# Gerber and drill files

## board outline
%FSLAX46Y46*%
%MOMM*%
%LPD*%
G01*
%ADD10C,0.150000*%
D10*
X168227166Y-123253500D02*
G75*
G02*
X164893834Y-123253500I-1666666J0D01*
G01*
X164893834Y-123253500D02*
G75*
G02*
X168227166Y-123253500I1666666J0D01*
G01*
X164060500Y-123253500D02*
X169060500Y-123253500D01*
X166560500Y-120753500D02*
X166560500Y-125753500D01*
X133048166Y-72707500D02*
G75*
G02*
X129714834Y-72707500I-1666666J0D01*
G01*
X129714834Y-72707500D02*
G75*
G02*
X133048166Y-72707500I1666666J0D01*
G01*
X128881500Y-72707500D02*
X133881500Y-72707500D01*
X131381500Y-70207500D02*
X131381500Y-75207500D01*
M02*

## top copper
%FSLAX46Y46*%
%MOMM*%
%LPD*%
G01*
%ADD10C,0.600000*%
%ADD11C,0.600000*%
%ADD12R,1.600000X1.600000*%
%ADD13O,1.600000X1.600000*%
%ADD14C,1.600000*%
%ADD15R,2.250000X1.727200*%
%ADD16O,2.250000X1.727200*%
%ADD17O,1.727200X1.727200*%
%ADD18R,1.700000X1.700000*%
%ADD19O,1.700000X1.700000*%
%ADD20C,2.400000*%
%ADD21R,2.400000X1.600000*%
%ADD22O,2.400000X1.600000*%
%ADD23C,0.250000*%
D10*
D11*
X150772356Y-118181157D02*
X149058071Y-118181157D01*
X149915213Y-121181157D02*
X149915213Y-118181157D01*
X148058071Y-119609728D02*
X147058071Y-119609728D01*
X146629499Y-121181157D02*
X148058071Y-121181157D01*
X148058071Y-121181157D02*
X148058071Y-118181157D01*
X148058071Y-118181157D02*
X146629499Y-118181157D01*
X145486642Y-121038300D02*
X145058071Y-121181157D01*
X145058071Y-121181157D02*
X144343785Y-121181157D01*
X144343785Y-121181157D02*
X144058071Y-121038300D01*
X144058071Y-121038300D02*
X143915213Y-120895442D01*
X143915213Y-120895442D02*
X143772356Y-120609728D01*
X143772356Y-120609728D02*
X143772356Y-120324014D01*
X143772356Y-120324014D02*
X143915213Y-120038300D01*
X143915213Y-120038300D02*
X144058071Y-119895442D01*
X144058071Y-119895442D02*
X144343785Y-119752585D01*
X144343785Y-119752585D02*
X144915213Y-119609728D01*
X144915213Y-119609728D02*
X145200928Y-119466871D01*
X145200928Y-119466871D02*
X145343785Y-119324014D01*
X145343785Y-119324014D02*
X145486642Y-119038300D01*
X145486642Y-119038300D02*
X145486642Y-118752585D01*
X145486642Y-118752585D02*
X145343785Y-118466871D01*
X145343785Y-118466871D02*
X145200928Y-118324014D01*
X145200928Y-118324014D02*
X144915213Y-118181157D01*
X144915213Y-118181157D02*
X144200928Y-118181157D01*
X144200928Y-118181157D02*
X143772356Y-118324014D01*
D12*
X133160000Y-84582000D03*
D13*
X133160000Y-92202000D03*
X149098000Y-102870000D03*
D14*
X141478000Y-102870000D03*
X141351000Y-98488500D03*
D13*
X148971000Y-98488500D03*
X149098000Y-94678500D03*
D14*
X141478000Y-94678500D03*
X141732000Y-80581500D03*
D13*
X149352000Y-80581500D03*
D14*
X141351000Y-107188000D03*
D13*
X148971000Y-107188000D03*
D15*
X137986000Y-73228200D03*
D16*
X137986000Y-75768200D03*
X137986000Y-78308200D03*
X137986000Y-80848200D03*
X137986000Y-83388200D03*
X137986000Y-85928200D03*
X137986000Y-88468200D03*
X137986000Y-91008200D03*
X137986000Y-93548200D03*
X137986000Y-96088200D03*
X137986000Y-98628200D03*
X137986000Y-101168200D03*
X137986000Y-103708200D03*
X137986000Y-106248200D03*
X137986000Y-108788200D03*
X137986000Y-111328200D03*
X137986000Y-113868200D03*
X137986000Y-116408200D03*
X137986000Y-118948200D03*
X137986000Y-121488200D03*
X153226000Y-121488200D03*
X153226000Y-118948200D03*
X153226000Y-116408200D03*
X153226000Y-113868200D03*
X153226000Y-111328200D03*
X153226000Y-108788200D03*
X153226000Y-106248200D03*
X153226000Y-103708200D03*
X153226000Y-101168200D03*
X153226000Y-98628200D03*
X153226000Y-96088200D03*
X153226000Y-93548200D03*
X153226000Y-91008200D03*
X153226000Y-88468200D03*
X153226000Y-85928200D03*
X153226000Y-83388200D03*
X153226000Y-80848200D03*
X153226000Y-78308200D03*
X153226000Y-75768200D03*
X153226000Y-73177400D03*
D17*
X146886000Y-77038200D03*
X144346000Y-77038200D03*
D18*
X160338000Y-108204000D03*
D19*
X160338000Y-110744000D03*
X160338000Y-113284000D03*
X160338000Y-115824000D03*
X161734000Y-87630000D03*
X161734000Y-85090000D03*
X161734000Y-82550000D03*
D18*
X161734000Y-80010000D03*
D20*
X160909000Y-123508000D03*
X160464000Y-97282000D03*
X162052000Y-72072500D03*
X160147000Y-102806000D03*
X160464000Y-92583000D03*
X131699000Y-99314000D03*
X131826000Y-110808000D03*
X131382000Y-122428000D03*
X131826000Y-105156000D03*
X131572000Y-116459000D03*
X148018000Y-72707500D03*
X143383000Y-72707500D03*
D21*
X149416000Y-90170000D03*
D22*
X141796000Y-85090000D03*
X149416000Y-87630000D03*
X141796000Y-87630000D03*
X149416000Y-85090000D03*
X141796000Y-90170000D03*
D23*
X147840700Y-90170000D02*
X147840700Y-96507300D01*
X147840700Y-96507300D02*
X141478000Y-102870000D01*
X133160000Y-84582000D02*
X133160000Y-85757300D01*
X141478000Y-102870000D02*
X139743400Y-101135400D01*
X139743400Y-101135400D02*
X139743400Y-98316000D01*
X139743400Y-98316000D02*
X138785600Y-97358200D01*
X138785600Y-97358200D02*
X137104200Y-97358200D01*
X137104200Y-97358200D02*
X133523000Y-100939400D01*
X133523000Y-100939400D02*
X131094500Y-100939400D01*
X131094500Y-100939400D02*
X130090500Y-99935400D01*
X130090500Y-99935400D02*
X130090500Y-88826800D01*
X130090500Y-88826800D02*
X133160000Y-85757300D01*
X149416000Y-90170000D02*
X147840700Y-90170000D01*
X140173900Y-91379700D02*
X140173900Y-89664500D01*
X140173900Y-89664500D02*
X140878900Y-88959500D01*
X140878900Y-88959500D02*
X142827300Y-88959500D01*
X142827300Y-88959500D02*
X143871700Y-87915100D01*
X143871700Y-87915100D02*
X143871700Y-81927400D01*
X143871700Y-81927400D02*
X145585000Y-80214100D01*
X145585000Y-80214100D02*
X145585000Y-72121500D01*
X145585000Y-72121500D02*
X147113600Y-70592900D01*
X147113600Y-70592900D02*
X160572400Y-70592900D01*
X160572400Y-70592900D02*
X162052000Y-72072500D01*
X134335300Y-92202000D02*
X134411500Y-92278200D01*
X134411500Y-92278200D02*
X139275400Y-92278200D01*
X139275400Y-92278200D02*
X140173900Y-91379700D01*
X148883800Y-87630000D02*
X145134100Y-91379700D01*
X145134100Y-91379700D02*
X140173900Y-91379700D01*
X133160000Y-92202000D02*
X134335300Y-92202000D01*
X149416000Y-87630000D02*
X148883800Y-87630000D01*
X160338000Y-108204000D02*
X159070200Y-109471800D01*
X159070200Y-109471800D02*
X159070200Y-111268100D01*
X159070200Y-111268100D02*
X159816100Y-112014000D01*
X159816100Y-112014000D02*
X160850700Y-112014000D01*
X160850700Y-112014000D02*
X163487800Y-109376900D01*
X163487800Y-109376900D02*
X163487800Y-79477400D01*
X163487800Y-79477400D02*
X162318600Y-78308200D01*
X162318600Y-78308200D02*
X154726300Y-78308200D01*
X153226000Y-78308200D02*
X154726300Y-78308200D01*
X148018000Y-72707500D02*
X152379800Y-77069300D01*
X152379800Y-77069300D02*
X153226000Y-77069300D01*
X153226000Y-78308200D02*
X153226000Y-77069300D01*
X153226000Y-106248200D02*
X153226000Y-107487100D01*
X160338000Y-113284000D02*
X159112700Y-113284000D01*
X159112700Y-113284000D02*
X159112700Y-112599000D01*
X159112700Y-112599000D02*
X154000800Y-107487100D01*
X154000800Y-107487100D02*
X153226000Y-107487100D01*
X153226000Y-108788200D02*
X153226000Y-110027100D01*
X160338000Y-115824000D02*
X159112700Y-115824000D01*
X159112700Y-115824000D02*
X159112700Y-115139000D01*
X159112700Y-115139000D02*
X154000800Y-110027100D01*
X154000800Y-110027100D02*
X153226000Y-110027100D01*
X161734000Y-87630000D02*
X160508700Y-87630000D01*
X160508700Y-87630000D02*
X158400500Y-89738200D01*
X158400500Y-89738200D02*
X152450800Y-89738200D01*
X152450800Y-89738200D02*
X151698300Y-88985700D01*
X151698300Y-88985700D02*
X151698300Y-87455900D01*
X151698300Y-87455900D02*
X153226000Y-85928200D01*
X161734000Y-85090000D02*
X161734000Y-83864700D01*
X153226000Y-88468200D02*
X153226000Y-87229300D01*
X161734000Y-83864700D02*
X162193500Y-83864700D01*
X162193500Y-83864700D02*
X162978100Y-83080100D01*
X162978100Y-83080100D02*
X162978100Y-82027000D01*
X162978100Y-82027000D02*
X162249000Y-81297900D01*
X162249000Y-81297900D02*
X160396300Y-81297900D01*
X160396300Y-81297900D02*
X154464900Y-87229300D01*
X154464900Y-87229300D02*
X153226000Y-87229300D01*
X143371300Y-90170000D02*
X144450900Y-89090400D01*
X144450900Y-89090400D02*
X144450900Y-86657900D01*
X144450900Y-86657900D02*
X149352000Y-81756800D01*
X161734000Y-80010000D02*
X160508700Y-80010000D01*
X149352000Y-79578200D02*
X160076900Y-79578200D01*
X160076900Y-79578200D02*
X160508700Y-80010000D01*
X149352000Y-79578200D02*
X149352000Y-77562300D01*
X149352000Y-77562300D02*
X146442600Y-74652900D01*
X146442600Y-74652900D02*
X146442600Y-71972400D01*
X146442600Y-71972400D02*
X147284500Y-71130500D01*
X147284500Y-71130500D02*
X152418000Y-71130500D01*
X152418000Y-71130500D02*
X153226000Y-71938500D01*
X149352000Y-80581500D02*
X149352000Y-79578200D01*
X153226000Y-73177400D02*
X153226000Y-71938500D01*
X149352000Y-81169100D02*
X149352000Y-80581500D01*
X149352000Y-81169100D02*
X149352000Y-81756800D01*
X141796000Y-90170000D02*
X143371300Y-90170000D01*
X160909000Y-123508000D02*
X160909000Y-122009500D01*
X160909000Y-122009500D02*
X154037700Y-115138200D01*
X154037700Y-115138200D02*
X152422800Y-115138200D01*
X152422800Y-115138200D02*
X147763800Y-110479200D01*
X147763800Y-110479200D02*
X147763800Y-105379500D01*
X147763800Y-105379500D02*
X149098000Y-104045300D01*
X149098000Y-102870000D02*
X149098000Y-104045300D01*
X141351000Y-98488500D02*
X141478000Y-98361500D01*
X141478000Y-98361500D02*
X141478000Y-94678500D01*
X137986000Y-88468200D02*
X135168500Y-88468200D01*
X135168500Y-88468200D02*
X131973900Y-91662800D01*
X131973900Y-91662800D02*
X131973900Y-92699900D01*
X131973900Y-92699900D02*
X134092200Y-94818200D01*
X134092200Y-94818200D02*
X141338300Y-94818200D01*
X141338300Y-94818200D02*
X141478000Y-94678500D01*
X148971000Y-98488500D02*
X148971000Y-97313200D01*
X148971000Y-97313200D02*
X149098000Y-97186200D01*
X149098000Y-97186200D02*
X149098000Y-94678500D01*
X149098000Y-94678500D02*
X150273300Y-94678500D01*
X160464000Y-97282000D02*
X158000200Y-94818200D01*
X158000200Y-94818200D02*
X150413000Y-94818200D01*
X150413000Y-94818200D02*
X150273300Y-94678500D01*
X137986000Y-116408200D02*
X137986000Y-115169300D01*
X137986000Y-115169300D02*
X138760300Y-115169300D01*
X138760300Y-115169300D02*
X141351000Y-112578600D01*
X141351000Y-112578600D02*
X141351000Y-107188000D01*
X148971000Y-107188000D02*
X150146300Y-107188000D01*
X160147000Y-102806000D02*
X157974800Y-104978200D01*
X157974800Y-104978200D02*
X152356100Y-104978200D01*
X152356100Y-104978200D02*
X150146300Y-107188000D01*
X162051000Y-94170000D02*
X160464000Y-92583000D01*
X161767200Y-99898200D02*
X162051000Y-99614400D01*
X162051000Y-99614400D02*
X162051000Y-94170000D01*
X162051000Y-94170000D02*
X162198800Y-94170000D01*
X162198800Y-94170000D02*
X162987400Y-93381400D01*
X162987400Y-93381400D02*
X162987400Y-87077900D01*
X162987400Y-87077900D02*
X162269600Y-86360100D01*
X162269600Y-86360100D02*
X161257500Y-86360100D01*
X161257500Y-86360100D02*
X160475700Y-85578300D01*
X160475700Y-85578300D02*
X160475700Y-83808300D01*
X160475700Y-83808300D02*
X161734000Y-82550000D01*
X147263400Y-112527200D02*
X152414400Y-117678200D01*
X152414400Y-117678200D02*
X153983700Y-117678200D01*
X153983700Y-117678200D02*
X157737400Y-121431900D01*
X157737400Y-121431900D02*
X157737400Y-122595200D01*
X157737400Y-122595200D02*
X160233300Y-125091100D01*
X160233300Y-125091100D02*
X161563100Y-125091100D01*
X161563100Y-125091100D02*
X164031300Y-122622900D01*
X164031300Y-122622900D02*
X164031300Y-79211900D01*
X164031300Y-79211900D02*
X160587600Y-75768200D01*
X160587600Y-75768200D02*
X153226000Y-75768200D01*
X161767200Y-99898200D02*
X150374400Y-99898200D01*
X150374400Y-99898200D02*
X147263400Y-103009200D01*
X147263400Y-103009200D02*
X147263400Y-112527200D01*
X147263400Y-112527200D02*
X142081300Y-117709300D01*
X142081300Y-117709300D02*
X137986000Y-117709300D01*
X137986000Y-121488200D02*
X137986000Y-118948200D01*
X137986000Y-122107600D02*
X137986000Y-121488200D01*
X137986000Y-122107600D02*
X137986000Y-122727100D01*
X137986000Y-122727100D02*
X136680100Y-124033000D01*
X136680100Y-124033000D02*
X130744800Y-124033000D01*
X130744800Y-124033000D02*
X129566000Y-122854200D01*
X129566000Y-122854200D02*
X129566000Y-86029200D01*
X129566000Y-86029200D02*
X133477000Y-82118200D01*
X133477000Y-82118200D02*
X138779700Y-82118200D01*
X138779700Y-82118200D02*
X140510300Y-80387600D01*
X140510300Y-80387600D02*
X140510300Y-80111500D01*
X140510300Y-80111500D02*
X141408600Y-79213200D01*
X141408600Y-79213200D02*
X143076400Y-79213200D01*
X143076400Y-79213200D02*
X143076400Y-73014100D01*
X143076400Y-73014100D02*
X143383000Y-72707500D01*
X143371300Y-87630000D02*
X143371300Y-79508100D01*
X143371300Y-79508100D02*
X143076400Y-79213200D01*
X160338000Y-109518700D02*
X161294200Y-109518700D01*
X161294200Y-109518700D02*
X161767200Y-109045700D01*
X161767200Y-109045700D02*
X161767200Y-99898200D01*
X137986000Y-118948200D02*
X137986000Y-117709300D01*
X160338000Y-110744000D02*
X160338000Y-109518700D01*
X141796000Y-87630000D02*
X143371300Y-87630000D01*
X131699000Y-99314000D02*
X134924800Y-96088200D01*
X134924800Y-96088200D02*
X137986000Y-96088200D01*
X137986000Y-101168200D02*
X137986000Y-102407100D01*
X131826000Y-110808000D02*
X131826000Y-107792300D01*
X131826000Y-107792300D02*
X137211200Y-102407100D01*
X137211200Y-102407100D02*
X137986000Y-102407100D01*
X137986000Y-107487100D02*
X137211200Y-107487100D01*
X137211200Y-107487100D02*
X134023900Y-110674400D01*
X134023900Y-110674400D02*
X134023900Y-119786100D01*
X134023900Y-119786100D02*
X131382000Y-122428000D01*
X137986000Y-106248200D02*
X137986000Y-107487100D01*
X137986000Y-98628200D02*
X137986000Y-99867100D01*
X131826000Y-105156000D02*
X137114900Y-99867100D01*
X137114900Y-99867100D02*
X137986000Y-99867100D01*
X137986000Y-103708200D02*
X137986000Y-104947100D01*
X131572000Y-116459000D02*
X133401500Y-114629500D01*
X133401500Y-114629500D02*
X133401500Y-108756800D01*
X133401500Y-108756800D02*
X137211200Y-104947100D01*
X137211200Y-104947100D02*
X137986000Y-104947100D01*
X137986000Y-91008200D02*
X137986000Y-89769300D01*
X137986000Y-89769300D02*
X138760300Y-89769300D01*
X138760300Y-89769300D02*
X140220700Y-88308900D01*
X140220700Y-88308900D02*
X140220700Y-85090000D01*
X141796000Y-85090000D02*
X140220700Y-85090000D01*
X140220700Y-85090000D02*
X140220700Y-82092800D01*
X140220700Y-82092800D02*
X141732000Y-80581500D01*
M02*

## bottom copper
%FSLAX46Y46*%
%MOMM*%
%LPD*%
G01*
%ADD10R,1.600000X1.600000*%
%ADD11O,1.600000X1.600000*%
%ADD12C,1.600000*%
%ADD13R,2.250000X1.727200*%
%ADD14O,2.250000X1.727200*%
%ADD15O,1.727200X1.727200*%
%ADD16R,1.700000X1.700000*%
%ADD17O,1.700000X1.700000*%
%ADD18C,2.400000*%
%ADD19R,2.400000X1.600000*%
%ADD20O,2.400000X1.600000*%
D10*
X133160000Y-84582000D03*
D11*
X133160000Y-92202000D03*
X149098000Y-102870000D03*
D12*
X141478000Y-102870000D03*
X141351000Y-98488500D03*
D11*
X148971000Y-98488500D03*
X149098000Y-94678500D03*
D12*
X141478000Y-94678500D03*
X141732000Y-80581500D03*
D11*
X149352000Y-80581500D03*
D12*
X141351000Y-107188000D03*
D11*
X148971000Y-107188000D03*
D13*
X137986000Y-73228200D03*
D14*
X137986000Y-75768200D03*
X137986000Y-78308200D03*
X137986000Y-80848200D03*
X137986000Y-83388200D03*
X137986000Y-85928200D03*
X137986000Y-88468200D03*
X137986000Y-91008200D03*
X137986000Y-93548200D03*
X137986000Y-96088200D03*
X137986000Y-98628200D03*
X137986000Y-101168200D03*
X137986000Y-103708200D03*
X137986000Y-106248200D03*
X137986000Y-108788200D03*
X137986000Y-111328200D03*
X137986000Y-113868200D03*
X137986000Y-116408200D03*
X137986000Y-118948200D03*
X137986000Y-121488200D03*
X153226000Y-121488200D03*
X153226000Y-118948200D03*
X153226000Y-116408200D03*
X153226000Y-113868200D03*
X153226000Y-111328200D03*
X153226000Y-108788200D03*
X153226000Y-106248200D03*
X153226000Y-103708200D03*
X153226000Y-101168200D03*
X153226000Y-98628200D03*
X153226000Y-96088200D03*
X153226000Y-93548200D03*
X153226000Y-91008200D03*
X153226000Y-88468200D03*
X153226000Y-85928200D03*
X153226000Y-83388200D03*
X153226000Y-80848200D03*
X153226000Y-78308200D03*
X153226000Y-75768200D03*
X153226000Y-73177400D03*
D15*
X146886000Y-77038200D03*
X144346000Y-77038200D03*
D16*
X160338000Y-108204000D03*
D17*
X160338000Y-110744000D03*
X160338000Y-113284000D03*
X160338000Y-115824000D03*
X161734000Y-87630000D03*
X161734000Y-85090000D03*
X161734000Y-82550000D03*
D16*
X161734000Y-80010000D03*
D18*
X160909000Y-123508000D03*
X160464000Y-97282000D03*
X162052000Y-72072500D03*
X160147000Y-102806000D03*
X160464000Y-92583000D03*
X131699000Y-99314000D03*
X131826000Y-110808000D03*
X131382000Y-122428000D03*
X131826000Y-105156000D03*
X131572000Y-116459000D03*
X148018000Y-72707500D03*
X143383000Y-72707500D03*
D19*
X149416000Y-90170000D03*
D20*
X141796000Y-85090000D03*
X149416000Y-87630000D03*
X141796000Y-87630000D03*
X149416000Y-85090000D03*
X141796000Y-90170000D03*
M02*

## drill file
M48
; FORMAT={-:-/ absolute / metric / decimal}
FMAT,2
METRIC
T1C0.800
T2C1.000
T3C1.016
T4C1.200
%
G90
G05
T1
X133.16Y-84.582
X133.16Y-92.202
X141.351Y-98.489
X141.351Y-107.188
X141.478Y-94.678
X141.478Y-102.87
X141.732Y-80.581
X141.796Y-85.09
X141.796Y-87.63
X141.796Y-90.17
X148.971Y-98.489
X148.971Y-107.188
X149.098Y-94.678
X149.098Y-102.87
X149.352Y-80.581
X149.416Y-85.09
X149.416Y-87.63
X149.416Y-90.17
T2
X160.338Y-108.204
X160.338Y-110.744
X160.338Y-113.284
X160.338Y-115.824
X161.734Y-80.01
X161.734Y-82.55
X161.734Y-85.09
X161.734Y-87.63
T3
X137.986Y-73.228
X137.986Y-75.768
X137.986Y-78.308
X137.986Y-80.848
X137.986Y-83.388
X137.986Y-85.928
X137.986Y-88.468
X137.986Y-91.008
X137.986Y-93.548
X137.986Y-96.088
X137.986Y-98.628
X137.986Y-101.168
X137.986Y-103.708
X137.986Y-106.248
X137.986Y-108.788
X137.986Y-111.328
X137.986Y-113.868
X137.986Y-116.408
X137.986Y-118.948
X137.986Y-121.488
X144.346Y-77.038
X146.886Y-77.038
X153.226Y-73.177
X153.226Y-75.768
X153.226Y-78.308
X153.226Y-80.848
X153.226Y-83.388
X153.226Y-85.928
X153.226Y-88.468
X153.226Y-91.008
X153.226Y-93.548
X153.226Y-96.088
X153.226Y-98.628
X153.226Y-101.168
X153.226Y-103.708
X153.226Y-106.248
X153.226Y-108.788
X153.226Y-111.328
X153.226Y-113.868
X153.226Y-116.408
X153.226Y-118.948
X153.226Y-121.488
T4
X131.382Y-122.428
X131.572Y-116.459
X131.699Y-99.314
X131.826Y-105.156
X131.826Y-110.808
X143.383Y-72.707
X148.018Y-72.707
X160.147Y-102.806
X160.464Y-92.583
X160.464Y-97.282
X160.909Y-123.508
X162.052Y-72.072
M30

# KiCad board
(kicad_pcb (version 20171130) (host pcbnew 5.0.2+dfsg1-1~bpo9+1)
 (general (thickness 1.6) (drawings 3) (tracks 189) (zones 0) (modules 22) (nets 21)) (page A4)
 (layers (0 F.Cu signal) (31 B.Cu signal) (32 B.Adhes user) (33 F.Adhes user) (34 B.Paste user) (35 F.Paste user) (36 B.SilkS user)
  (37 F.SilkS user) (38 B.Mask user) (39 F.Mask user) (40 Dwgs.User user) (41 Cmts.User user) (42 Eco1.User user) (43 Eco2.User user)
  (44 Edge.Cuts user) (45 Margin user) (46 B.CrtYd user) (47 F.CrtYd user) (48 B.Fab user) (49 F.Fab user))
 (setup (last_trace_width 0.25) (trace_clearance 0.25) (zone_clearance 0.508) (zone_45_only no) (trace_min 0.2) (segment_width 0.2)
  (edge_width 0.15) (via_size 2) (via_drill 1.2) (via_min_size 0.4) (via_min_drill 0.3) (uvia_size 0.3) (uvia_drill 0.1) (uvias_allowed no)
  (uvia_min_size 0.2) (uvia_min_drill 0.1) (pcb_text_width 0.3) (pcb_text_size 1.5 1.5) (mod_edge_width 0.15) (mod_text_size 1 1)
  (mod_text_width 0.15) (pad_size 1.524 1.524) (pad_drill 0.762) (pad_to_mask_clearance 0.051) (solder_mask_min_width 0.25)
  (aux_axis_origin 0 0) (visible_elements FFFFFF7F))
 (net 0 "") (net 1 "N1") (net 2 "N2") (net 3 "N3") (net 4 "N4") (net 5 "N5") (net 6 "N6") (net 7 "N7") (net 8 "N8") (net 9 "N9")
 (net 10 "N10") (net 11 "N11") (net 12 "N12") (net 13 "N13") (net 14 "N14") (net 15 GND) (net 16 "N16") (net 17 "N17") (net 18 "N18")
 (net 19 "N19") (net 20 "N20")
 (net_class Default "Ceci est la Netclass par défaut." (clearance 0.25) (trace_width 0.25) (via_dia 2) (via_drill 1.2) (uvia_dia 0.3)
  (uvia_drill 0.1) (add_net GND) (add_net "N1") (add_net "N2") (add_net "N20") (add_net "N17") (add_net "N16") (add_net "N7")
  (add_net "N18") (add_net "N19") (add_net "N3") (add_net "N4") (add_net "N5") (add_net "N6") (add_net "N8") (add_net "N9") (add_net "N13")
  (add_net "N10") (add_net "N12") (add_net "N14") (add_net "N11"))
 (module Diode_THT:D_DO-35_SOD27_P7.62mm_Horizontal (layer F.Cu) (at 133.16 84.582 270)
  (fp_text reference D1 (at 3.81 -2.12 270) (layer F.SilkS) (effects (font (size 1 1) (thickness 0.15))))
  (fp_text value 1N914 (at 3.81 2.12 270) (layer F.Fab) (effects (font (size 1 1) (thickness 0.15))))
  (pad 1 thru_hole rect (at 0 0 270) (size 1.6 1.6) (drill 0.8) (layers *.Cu *.Mask) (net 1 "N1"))
  (pad 2 thru_hole oval (at 7.62 0 270) (size 1.6 1.6) (drill 0.8) (layers *.Cu *.Mask) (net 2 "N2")))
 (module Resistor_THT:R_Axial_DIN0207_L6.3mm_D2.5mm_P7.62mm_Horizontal (layer F.Cu) (at 141.478 102.87)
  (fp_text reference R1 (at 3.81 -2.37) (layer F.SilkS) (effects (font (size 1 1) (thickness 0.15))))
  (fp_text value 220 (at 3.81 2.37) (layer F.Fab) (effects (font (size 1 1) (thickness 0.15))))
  (pad 2 thru_hole oval (at 7.62 0) (size 1.6 1.6) (drill 0.8) (layers *.Cu *.Mask) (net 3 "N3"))
  (pad 1 thru_hole circle (at 0 0) (size 1.6 1.6) (drill 0.8) (layers *.Cu *.Mask) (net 1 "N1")))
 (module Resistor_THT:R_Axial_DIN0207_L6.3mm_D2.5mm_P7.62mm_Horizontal (layer F.Cu) (at 141.351 98.4885)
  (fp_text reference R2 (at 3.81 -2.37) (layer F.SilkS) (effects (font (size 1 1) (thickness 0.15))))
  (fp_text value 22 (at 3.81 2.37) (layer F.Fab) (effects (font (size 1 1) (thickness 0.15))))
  (pad 1 thru_hole circle (at 0 0) (size 1.6 1.6) (drill 0.8) (layers *.Cu *.Mask) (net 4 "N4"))
  (pad 2 thru_hole oval (at 7.62 0) (size 1.6 1.6) (drill 0.8) (layers *.Cu *.Mask) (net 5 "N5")))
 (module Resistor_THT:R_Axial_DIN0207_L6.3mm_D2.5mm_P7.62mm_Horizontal (layer F.Cu) (at 141.478 94.6785)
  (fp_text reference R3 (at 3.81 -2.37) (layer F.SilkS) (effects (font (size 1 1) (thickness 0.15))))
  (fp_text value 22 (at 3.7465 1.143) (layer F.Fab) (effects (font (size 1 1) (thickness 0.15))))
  (pad 2 thru_hole oval (at 7.62 0) (size 1.6 1.6) (drill 0.8) (layers *.Cu *.Mask) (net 5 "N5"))
  (pad 1 thru_hole circle (at 0 0) (size 1.6 1.6) (drill 0.8) (layers *.Cu *.Mask) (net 4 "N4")))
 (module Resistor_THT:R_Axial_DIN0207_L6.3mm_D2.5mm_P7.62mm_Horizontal (layer F.Cu) (at 141.732 80.5815)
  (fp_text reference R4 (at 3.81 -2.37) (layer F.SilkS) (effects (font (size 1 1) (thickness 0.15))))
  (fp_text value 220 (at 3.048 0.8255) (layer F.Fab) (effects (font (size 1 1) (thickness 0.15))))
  (pad 1 thru_hole circle (at 0 0) (size 1.6 1.6) (drill 0.8) (layers *.Cu *.Mask) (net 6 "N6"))
  (pad 2 thru_hole oval (at 7.62 0) (size 1.6 1.6) (drill 0.8) (layers *.Cu *.Mask) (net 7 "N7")))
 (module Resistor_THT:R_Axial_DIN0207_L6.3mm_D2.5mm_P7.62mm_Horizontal (layer F.Cu) (at 141.351 107.188)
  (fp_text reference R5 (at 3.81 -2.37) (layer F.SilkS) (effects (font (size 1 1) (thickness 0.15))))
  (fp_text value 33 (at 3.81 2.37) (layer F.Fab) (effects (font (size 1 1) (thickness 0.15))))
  (pad 1 thru_hole circle (at 0 0) (size 1.6 1.6) (drill 0.8) (layers *.Cu *.Mask) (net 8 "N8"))
  (pad 2 thru_hole oval (at 7.62 0) (size 1.6 1.6) (drill 0.8) (layers *.Cu *.Mask) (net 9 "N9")))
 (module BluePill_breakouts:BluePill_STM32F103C (layer F.Cu) (at 137.986 73.279)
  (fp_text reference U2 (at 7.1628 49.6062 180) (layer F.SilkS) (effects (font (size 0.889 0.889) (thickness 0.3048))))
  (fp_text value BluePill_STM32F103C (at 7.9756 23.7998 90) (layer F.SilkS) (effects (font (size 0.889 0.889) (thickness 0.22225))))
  (pad 1 thru_hole rect (at 0 -0.0508 270) (size 1.7272 2.25) (drill 1.016) (layers *.Cu *.Mask F.SilkS))
  (pad 2 thru_hole oval (at 0 2.4892 270) (size 1.7272 2.25) (drill 1.016) (layers *.Cu *.Mask F.SilkS))
  (pad 3 thru_hole oval (at 0 5.0292 270) (size 1.7272 2.25) (drill 1.016) (layers *.Cu *.Mask F.SilkS))
  (pad 4 thru_hole oval (at 0 7.5692 270) (size 1.7272 2.25) (drill 1.016) (layers *.Cu *.Mask F.SilkS))
  (pad 5 thru_hole oval (at 0 10.1092 270) (size 1.7272 2.25) (drill 1.016) (layers *.Cu *.Mask F.SilkS))
  (pad 6 thru_hole oval (at 0 12.6492 270) (size 1.7272 2.25) (drill 1.016) (layers *.Cu *.Mask F.SilkS))
  (pad 7 thru_hole oval (at 0 15.1892 270) (size 1.7272 2.25) (drill 1.016) (layers *.Cu *.Mask F.SilkS) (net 4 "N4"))
  (pad 8 thru_hole oval (at 0 17.7292 270) (size 1.7272 2.25) (drill 1.016) (layers *.Cu *.Mask F.SilkS) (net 6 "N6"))
  (pad 9 thru_hole oval (at 0 20.2692 270) (size 1.7272 2.25) (drill 1.016) (layers *.Cu *.Mask F.SilkS))
  (pad 10 thru_hole oval (at 0 22.8092 270) (size 1.7272 2.25) (drill 1.016) (layers *.Cu *.Mask F.SilkS) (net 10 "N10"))
  (pad 11 thru_hole oval (at 0 25.3492 270) (size 1.7272 2.25) (drill 1.016) (layers *.Cu *.Mask F.SilkS) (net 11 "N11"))
  (pad 12 thru_hole oval (at 0 27.8892 270) (size 1.7272 2.25) (drill 1.016) (layers *.Cu *.Mask F.SilkS) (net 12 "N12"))
  (pad 13 thru_hole oval (at 0 30.4292 270) (size 1.7272 2.25) (drill 1.016) (layers *.Cu *.Mask F.SilkS) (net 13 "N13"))
  (pad 14 thru_hole oval (at 0 32.9692 270) (size 1.7272 2.25) (drill 1.016) (layers *.Cu *.Mask F.SilkS) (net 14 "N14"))
  (pad 15 thru_hole oval (at 0 35.5092 270) (size 1.7272 2.25) (drill 1.016) (layers *.Cu *.Mask F.SilkS))
  (pad 16 thru_hole oval (at 0 38.0492 270) (size 1.7272 2.25) (drill 1.016) (layers *.Cu *.Mask F.SilkS))
  (pad 17 thru_hole oval (at 0 40.5892 270) (size 1.7272 2.25) (drill 1.016) (layers *.Cu *.Mask F.SilkS))
  (pad 18 thru_hole oval (at 0 43.1292 270) (size 1.7272 2.25) (drill 1.016) (layers *.Cu *.Mask F.SilkS) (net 8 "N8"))
  (pad 19 thru_hole oval (at 0 45.6692 270) (size 1.7272 2.25) (drill 1.016) (layers *.Cu *.Mask F.SilkS) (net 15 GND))
  (pad 20 thru_hole oval (at 0 48.2092 270) (size 1.7272 2.25) (drill 1.016) (layers *.Cu *.Mask F.SilkS) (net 15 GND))
  (pad 21 thru_hole oval (at 15.24 48.2092 90) (size 1.7272 2.25) (drill 1.016) (layers *.Cu *.Mask F.SilkS))
  (pad 22 thru_hole oval (at 15.24 45.6692 90) (size 1.7272 2.25) (drill 1.016) (layers *.Cu *.Mask F.SilkS))
  (pad 23 thru_hole oval (at 15.24 43.1292 90) (size 1.7272 2.25) (drill 1.016) (layers *.Cu *.Mask F.SilkS))
  (pad 24 thru_hole oval (at 15.24 40.5892 90) (size 1.7272 2.25) (drill 1.016) (layers *.Cu *.Mask F.SilkS))
  (pad 25 thru_hole oval (at 15.24 38.0492 90) (size 1.7272 2.25) (drill 1.016) (layers *.Cu *.Mask F.SilkS))
  (pad 26 thru_hole oval (at 15.24 35.5092 90) (size 1.7272 2.25) (drill 1.016) (layers *.Cu *.Mask F.SilkS) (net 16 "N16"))
  (pad 27 thru_hole oval (at 15.24 32.9692 90) (size 1.7272 2.25) (drill 1.016) (layers *.Cu *.Mask F.SilkS) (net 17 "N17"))
  (pad 28 thru_hole oval (at 15.24 30.4292 90) (size 1.7272 2.25) (drill 1.016) (layers *.Cu *.Mask F.SilkS))
  (pad 29 thru_hole oval (at 15.24 27.8892 90) (size 1.7272 2.25) (drill 1.016) (layers *.Cu *.Mask F.SilkS))
  (pad 30 thru_hole oval (at 15.24 25.3492 90) (size 1.7272 2.25) (drill 1.016) (layers *.Cu *.Mask F.SilkS))
  (pad 31 thru_hole oval (at 15.24 22.8092 90) (size 1.7272 2.25) (drill 1.016) (layers *.Cu *.Mask F.SilkS))
  (pad 32 thru_hole oval (at 15.24 20.2692 90) (size 1.7272 2.25) (drill 1.016) (layers *.Cu *.Mask F.SilkS))
  (pad 33 thru_hole oval (at 15.24 17.7292 90) (size 1.7272 2.25) (drill 1.016) (layers *.Cu *.Mask F.SilkS))
  (pad 34 thru_hole oval (at 15.24 15.1892 90) (size 1.7272 2.25) (drill 1.016) (layers *.Cu *.Mask F.SilkS) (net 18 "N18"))
  (pad 35 thru_hole oval (at 15.24 12.6492 90) (size 1.7272 2.25) (drill 1.016) (layers *.Cu *.Mask F.SilkS) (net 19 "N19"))
  (pad 36 thru_hole oval (at 15.24 10.1092 90) (size 1.7272 2.25) (drill 1.016) (layers *.Cu *.Mask F.SilkS))
  (pad 37 thru_hole oval (at 15.24 7.5692 90) (size 1.7272 2.25) (drill 1.016) (layers *.Cu *.Mask F.SilkS))
  (pad 38 thru_hole oval (at 15.24 5.0292 90) (size 1.7272 2.25) (drill 1.016) (layers *.Cu *.Mask F.SilkS) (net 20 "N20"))
  (pad 39 thru_hole oval (at 15.24 2.4892 90) (size 1.7272 2.25) (drill 1.016) (layers *.Cu *.Mask F.SilkS) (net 15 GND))
  (pad 40 thru_hole oval (at 15.24 -0.1016 90) (size 1.7272 2.25) (drill 1.016) (layers *.Cu *.Mask F.SilkS) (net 7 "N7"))
  (pad 41 thru_hole oval (at 8.9 3.7592 90) (size 1.7272 1.7272) (drill 1.016) (layers *.Cu *.Mask F.SilkS))
  (pad 42 thru_hole oval (at 6.36 3.7592 90) (size 1.7272 1.7272) (drill 1.016) (layers *.Cu *.Mask F.SilkS)))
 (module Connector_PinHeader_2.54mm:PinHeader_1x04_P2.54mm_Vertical (layer F.Cu) (at 160.338 108.204)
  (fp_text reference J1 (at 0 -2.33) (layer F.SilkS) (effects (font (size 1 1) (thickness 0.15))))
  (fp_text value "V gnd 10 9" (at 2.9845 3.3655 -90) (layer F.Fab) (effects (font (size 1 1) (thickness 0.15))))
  (pad 1 thru_hole rect (at 0 0) (size 1.7 1.7) (drill 1) (layers *.Cu *.Mask) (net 20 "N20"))
  (pad 2 thru_hole oval (at 0 2.54) (size 1.7 1.7) (drill 1) (layers *.Cu *.Mask) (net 15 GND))
  (pad 3 thru_hole oval (at 0 5.08) (size 1.7 1.7) (drill 1) (layers *.Cu *.Mask) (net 17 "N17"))
  (pad 4 thru_hole oval (at 0 7.62) (size 1.7 1.7) (drill 1) (layers *.Cu *.Mask) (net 16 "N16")))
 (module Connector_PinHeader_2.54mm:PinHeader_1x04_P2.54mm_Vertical (layer F.Cu) (at 161.734 80.01)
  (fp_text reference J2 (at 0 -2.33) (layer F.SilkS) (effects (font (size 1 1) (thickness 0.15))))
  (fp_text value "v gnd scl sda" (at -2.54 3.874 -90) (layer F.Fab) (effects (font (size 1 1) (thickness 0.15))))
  (pad 4 thru_hole oval (at 0 7.62) (size 1.7 1.7) (drill 1) (layers *.Cu *.Mask) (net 19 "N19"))
  (pad 3 thru_hole oval (at 0 5.08) (size 1.7 1.7) (drill 1) (layers *.Cu *.Mask) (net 18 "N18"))
  (pad 2 thru_hole oval (at 0 2.54) (size 1.7 1.7) (drill 1) (layers *.Cu *.Mask) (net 15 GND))
  (pad 1 thru_hole rect (at 0 0) (size 1.7 1.7) (drill 1) (layers *.Cu *.Mask) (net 7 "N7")))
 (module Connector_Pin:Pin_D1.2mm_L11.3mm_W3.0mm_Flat (layer F.Cu) (at 160.909 123.508)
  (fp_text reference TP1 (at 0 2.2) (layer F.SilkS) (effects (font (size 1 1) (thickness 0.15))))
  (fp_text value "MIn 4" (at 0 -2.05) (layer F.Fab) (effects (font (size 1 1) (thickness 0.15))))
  (pad 1 thru_hole circle (at 0 0) (size 2.4 2.4) (drill 1.2) (layers *.Cu *.Mask) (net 3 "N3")))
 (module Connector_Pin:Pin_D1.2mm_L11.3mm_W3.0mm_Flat (layer F.Cu) (at 160.464 97.282)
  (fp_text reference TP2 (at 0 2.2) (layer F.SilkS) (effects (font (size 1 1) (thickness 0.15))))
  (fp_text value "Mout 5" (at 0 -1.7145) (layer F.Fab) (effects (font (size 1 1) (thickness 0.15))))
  (pad 1 thru_hole circle (at 0 0) (size 2.4 2.4) (drill 1.2) (layers *.Cu *.Mask) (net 5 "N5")))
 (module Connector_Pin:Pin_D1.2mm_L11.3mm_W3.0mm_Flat (layer F.Cu) (at 162.052 72.0725)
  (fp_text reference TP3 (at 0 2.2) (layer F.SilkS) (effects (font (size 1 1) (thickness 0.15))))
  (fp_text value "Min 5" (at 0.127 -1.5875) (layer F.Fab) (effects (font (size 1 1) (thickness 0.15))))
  (pad 1 thru_hole circle (at 0 0) (size 2.4 2.4) (drill 1.2) (layers *.Cu *.Mask) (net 2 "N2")))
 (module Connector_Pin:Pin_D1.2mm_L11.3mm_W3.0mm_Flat (layer F.Cu) (at 160.147 102.806)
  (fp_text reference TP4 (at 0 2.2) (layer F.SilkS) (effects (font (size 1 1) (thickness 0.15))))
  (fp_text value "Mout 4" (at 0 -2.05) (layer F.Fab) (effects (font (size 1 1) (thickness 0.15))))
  (pad 1 thru_hole circle (at 0 0) (size 2.4 2.4) (drill 1.2) (layers *.Cu *.Mask) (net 9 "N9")))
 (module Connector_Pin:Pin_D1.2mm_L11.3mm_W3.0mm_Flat (layer F.Cu) (at 160.464 92.583)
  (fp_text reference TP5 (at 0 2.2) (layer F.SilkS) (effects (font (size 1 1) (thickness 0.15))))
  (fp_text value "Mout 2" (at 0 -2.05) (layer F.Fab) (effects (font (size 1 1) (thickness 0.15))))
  (pad 1 thru_hole circle (at 0 0) (size 2.4 2.4) (drill 1.2) (layers *.Cu *.Mask) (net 15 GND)))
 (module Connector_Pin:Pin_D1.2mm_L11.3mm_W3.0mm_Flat (layer F.Cu) (at 131.699 99.314)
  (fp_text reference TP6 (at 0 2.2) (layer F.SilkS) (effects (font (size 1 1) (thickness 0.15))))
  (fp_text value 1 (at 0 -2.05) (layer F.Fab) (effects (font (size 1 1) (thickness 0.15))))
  (pad 1 thru_hole circle (at 0 0) (size 2.4 2.4) (drill 1.2) (layers *.Cu *.Mask) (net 10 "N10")))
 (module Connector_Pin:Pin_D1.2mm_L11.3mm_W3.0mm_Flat (layer F.Cu) (at 131.826 110.808)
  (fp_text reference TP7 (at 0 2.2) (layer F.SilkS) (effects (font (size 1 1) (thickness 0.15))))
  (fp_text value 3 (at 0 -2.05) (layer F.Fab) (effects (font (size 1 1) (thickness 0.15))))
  (pad 1 thru_hole circle (at 0 0) (size 2.4 2.4) (drill 1.2) (layers *.Cu *.Mask) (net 12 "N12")))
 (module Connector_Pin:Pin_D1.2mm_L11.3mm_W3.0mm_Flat (layer F.Cu) (at 131.382 122.428)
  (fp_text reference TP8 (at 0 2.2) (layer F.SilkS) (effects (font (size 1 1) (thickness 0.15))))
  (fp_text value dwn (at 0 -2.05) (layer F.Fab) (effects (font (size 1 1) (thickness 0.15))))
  (pad 1 thru_hole circle (at 0 0) (size 2.4 2.4) (drill 1.2) (layers *.Cu *.Mask) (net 14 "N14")))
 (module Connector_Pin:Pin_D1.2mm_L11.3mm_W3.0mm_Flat (layer F.Cu) (at 131.826 105.156)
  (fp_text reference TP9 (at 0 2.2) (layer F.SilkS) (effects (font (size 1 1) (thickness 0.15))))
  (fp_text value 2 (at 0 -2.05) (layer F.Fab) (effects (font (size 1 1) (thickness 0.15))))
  (pad 1 thru_hole circle (at 0 0) (size 2.4 2.4) (drill 1.2) (layers *.Cu *.Mask) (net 11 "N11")))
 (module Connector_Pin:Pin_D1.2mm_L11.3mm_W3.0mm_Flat (layer F.Cu) (at 131.572 116.459)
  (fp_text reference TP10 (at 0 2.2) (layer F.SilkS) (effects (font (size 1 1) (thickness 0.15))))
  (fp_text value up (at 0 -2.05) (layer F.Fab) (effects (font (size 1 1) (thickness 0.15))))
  (pad 1 thru_hole circle (at 0 0) (size 2.4 2.4) (drill 1.2) (layers *.Cu *.Mask) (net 13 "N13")))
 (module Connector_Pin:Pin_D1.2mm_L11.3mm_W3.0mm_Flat (layer F.Cu) (at 148.018 72.7075)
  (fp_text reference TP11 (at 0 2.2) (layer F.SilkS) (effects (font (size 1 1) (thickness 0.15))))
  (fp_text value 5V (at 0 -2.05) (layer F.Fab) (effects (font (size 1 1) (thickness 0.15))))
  (pad 1 thru_hole circle (at 0 0) (size 2.4 2.4) (drill 1.2) (layers *.Cu *.Mask) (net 20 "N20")))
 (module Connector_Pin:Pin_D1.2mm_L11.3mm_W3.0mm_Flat (layer F.Cu) (at 143.383 72.7075)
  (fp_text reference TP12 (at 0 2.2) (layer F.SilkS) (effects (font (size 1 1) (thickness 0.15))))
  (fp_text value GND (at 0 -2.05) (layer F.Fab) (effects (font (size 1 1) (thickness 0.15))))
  (pad 1 thru_hole circle (at 0 0) (size 2.4 2.4) (drill 1.2) (layers *.Cu *.Mask) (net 15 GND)))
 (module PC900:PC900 (layer F.Cu) (at 149.416 90.17 180)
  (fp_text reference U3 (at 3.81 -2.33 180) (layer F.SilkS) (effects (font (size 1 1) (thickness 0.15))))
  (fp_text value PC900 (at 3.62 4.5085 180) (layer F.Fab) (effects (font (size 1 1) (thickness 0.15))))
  (pad 1 thru_hole rect (at 0 0 180) (size 2.4 1.6) (drill 0.8) (layers *.Cu *.Mask) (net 1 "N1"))
  (pad 4 thru_hole oval (at 7.62 5.08 180) (size 2.4 1.6) (drill 0.8) (layers *.Cu *.Mask) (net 6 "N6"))
  (pad 2 thru_hole oval (at 0 2.54 180) (size 2.4 1.6) (drill 0.8) (layers *.Cu *.Mask) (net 2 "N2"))
  (pad 5 thru_hole oval (at 7.62 2.54 180) (size 2.4 1.6) (drill 0.8) (layers *.Cu *.Mask) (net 15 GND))
  (pad 3 thru_hole oval (at 0 5.08 180) (size 2.4 1.6) (drill 0.8) (layers *.Cu *.Mask))
  (pad 6 thru_hole oval (at 7.62 0 180) (size 2.4 1.6) (drill 0.8) (layers *.Cu *.Mask) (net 7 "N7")))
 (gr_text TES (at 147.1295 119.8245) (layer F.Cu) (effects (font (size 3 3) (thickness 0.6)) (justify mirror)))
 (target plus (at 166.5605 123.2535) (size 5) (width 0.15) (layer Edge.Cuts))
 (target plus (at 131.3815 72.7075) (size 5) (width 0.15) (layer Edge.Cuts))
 (segment (start 147.8407 90.17) (end 147.8407 96.5073) (width 0.25) (layer F.Cu) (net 1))
 (segment (start 147.8407 96.5073) (end 141.478 102.87) (width 0.25) (layer F.Cu) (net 1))
 (segment (start 133.16 84.582) (end 133.16 85.7573) (width 0.25) (layer F.Cu) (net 1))
 (segment (start 141.478 102.87) (end 139.7434 101.1354) (width 0.25) (layer F.Cu) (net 1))
 (segment (start 139.7434 101.1354) (end 139.7434 98.316) (width 0.25) (layer F.Cu) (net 1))
 (segment (start 139.7434 98.316) (end 138.7856 97.3582) (width 0.25) (layer F.Cu) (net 1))
 (segment (start 138.7856 97.3582) (end 137.1042 97.3582) (width 0.25) (layer F.Cu) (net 1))
 (segment (start 137.1042 97.3582) (end 133.523 100.9394) (width 0.25) (layer F.Cu) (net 1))
 (segment (start 133.523 100.9394) (end 131.0945 100.9394) (width 0.25) (layer F.Cu) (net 1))
 (segment (start 131.0945 100.9394) (end 130.0905 99.9354) (width 0.25) (layer F.Cu) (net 1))
 (segment (start 130.0905 99.9354) (end 130.0905 88.8268) (width 0.25) (layer F.Cu) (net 1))
 (segment (start 130.0905 88.8268) (end 133.16 85.7573) (width 0.25) (layer F.Cu) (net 1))
 (segment (start 149.416 90.17) (end 147.8407 90.17) (width 0.25) (layer F.Cu) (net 1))
 (segment (start 140.1739 91.3797) (end 140.1739 89.6645) (width 0.25) (layer F.Cu) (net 2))
 (segment (start 140.1739 89.6645) (end 140.8789 88.9595) (width 0.25) (layer F.Cu) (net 2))
 (segment (start 140.8789 88.9595) (end 142.8273 88.9595) (width 0.25) (layer F.Cu) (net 2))
 (segment (start 142.8273 88.9595) (end 143.8717 87.9151) (width 0.25) (layer F.Cu) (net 2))
 (segment (start 143.8717 87.9151) (end 143.8717 81.9274) (width 0.25) (layer F.Cu) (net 2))
 (segment (start 143.8717 81.9274) (end 145.585 80.2141) (width 0.25) (layer F.Cu) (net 2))
 (segment (start 145.585 80.2141) (end 145.585 72.1215) (width 0.25) (layer F.Cu) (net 2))
 (segment (start 145.585 72.1215) (end 147.1136 70.5929) (width 0.25) (layer F.Cu) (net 2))
 (segment (start 147.1136 70.5929) (end 160.5724 70.5929) (width 0.25) (layer F.Cu) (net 2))
 (segment (start 160.5724 70.5929) (end 162.052 72.0725) (width 0.25) (layer F.Cu) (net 2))
 (segment (start 134.3353 92.202) (end 134.4115 92.2782) (width 0.25) (layer F.Cu) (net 2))
 (segment (start 134.4115 92.2782) (end 139.2754 92.2782) (width 0.25) (layer F.Cu) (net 2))
 (segment (start 139.2754 92.2782) (end 140.1739 91.3797) (width 0.25) (layer F.Cu) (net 2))
 (segment (start 148.8838 87.63) (end 145.1341 91.3797) (width 0.25) (layer F.Cu) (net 2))
 (segment (start 145.1341 91.3797) (end 140.1739 91.3797) (width 0.25) (layer F.Cu) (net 2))
 (segment (start 133.16 92.202) (end 134.3353 92.202) (width 0.25) (layer F.Cu) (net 2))
 (segment (start 149.416 87.63) (end 148.8838 87.63) (width 0.25) (layer F.Cu) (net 2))
 (segment (start 160.338 108.204) (end 159.0702 109.4718) (width 0.25) (layer F.Cu) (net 20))
 (segment (start 159.0702 109.4718) (end 159.0702 111.2681) (width 0.25) (layer F.Cu) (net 20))
 (segment (start 159.0702 111.2681) (end 159.8161 112.014) (width 0.25) (layer F.Cu) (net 20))
 (segment (start 159.8161 112.014) (end 160.8507 112.014) (width 0.25) (layer F.Cu) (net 20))
 (segment (start 160.8507 112.014) (end 163.4878 109.3769) (width 0.25) (layer F.Cu) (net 20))
 (segment (start 163.4878 109.3769) (end 163.4878 79.4774) (width 0.25) (layer F.Cu) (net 20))
 (segment (start 163.4878 79.4774) (end 162.3186 78.3082) (width 0.25) (layer F.Cu) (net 20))
 (segment (start 162.3186 78.3082) (end 154.7263 78.3082) (width 0.25) (layer F.Cu) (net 20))
 (segment (start 153.226 78.3082) (end 154.7263 78.3082) (width 0.25) (layer F.Cu) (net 20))
 (segment (start 148.018 72.7075) (end 152.3798 77.0693) (width 0.25) (layer F.Cu) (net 20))
 (segment (start 152.3798 77.0693) (end 153.226 77.0693) (width 0.25) (layer F.Cu) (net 20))
 (segment (start 153.226 78.3082) (end 153.226 77.0693) (width 0.25) (layer F.Cu) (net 20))
 (segment (start 153.226 106.2482) (end 153.226 107.4871) (width 0.25) (layer F.Cu) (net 17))
 (segment (start 160.338 113.284) (end 159.1127 113.284) (width 0.25) (layer F.Cu) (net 17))
 (segment (start 159.1127 113.284) (end 159.1127 112.599) (width 0.25) (layer F.Cu) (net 17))
 (segment (start 159.1127 112.599) (end 154.0008 107.4871) (width 0.25) (layer F.Cu) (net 17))
 (segment (start 154.0008 107.4871) (end 153.226 107.4871) (width 0.25) (layer F.Cu) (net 17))
 (segment (start 153.226 108.7882) (end 153.226 110.0271) (width 0.25) (layer F.Cu) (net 16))
 (segment (start 160.338 115.824) (end 159.1127 115.824) (width 0.25) (layer F.Cu) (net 16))
 (segment (start 159.1127 115.824) (end 159.1127 115.139) (width 0.25) (layer F.Cu) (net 16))
 (segment (start 159.1127 115.139) (end 154.0008 110.0271) (width 0.25) (layer F.Cu) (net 16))
 (segment (start 154.0008 110.0271) (end 153.226 110.0271) (width 0.25) (layer F.Cu) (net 16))
 (segment (start 161.734 87.63) (end 160.5087 87.63) (width 0.25) (layer F.Cu) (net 19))
 (segment (start 160.5087 87.63) (end 158.4005 89.7382) (width 0.25) (layer F.Cu) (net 19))
 (segment (start 158.4005 89.7382) (end 152.4508 89.7382) (width 0.25) (layer F.Cu) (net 19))
 (segment (start 152.4508 89.7382) (end 151.6983 88.9857) (width 0.25) (layer F.Cu) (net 19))
 (segment (start 151.6983 88.9857) (end 151.6983 87.4559) (width 0.25) (layer F.Cu) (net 19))
 (segment (start 151.6983 87.4559) (end 153.226 85.9282) (width 0.25) (layer F.Cu) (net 19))
 (segment (start 161.734 85.09) (end 161.734 83.8647) (width 0.25) (layer F.Cu) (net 18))
 (segment (start 153.226 88.4682) (end 153.226 87.2293) (width 0.25) (layer F.Cu) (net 18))
 (segment (start 161.734 83.8647) (end 162.1935 83.8647) (width 0.25) (layer F.Cu) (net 18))
 (segment (start 162.1935 83.8647) (end 162.9781 83.0801) (width 0.25) (layer F.Cu) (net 18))
 (segment (start 162.9781 83.0801) (end 162.9781 82.027) (width 0.25) (layer F.Cu) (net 18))
 (segment (start 162.9781 82.027) (end 162.249 81.2979) (width 0.25) (layer F.Cu) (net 18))
 (segment (start 162.249 81.2979) (end 160.3963 81.2979) (width 0.25) (layer F.Cu) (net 18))
 (segment (start 160.3963 81.2979) (end 154.4649 87.2293) (width 0.25) (layer F.Cu) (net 18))
 (segment (start 154.4649 87.2293) (end 153.226 87.2293) (width 0.25) (layer F.Cu) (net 18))
 (segment (start 143.3713 90.17) (end 144.4509 89.0904) (width 0.25) (layer F.Cu) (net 7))
 (segment (start 144.4509 89.0904) (end 144.4509 86.6579) (width 0.25) (layer F.Cu) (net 7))
 (segment (start 144.4509 86.6579) (end 149.352 81.7568) (width 0.25) (layer F.Cu) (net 7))
 (segment (start 161.734 80.01) (end 160.5087 80.01) (width 0.25) (layer F.Cu) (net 7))
 (segment (start 149.352 79.5782) (end 160.0769 79.5782) (width 0.25) (layer F.Cu) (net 7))
 (segment (start 160.0769 79.5782) (end 160.5087 80.01) (width 0.25) (layer F.Cu) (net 7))
 (segment (start 149.352 79.5782) (end 149.352 77.5623) (width 0.25) (layer F.Cu) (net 7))
 (segment (start 149.352 77.5623) (end 146.4426 74.6529) (width 0.25) (layer F.Cu) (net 7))
 (segment (start 146.4426 74.6529) (end 146.4426 71.9724) (width 0.25) (layer F.Cu) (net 7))
 (segment (start 146.4426 71.9724) (end 147.2845 71.1305) (width 0.25) (layer F.Cu) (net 7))
 (segment (start 147.2845 71.1305) (end 152.418 71.1305) (width 0.25) (layer F.Cu) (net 7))
 (segment (start 152.418 71.1305) (end 153.226 71.9385) (width 0.25) (layer F.Cu) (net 7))
 (segment (start 149.352 80.5815) (end 149.352 79.5782) (width 0.25) (layer F.Cu) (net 7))
 (segment (start 153.226 73.1774) (end 153.226 71.9385) (width 0.25) (layer F.Cu) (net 7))
 (segment (start 149.352 81.1691) (end 149.352 80.5815) (width 0.25) (layer F.Cu) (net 7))
 (segment (start 149.352 81.1691) (end 149.352 81.7568) (width 0.25) (layer F.Cu) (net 7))
 (segment (start 141.796 90.17) (end 143.3713 90.17) (width 0.25) (layer F.Cu) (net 7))
 (segment (start 160.909 123.508) (end 160.909 122.0095) (width 0.25) (layer F.Cu) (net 3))
 (segment (start 160.909 122.0095) (end 154.0377 115.1382) (width 0.25) (layer F.Cu) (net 3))
 (segment (start 154.0377 115.1382) (end 152.4228 115.1382) (width 0.25) (layer F.Cu) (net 3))
 (segment (start 152.4228 115.1382) (end 147.7638 110.4792) (width 0.25) (layer F.Cu) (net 3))
 (segment (start 147.7638 110.4792) (end 147.7638 105.3795) (width 0.25) (layer F.Cu) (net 3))
 (segment (start 147.7638 105.3795) (end 149.098 104.0453) (width 0.25) (layer F.Cu) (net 3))
 (segment (start 149.098 102.87) (end 149.098 104.0453) (width 0.25) (layer F.Cu) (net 3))
 (segment (start 141.351 98.4885) (end 141.478 98.3615) (width 0.25) (layer F.Cu) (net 4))
 (segment (start 141.478 98.3615) (end 141.478 94.6785) (width 0.25) (layer F.Cu) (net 4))
 (segment (start 137.986 88.4682) (end 135.1685 88.4682) (width 0.25) (layer F.Cu) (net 4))
 (segment (start 135.1685 88.4682) (end 131.9739 91.6628) (width 0.25) (layer F.Cu) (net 4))
 (segment (start 131.9739 91.6628) (end 131.9739 92.6999) (width 0.25) (layer F.Cu) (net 4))
 (segment (start 131.9739 92.6999) (end 134.0922 94.8182) (width 0.25) (layer F.Cu) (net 4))
 (segment (start 134.0922 94.8182) (end 141.3383 94.8182) (width 0.25) (layer F.Cu) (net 4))
 (segment (start 141.3383 94.8182) (end 141.478 94.6785) (width 0.25) (layer F.Cu) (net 4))
 (segment (start 148.971 98.4885) (end 148.971 97.3132) (width 0.25) (layer F.Cu) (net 5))
 (segment (start 148.971 97.3132) (end 149.098 97.1862) (width 0.25) (layer F.Cu) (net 5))
 (segment (start 149.098 97.1862) (end 149.098 94.6785) (width 0.25) (layer F.Cu) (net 5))
 (segment (start 149.098 94.6785) (end 150.2733 94.6785) (width 0.25) (layer F.Cu) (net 5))
 (segment (start 160.464 97.282) (end 158.0002 94.8182) (width 0.25) (layer F.Cu) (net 5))
 (segment (start 158.0002 94.8182) (end 150.413 94.8182) (width 0.25) (layer F.Cu) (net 5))
 (segment (start 150.413 94.8182) (end 150.2733 94.6785) (width 0.25) (layer F.Cu) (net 5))
 (segment (start 137.986 116.4082) (end 137.986 115.1693) (width 0.25) (layer F.Cu) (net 8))
 (segment (start 137.986 115.1693) (end 138.7603 115.1693) (width 0.25) (layer F.Cu) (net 8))
 (segment (start 138.7603 115.1693) (end 141.351 112.5786) (width 0.25) (layer F.Cu) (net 8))
 (segment (start 141.351 112.5786) (end 141.351 107.188) (width 0.25) (layer F.Cu) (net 8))
 (segment (start 148.971 107.188) (end 150.1463 107.188) (width 0.25) (layer F.Cu) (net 9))
 (segment (start 160.147 102.806) (end 157.9748 104.9782) (width 0.25) (layer F.Cu) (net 9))
 (segment (start 157.9748 104.9782) (end 152.3561 104.9782) (width 0.25) (layer F.Cu) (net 9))
 (segment (start 152.3561 104.9782) (end 150.1463 107.188) (width 0.25) (layer F.Cu) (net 9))
 (segment (start 162.051 94.17) (end 160.464 92.583) (width 0.25) (layer F.Cu) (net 15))
 (segment (start 161.7672 99.8982) (end 162.051 99.6144) (width 0.25) (layer F.Cu) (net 15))
 (segment (start 162.051 99.6144) (end 162.051 94.17) (width 0.25) (layer F.Cu) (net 15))
 (segment (start 162.051 94.17) (end 162.1988 94.17) (width 0.25) (layer F.Cu) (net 15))
 (segment (start 162.1988 94.17) (end 162.9874 93.3814) (width 0.25) (layer F.Cu) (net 15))
 (segment (start 162.9874 93.3814) (end 162.9874 87.0779) (width 0.25) (layer F.Cu) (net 15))
 (segment (start 162.9874 87.0779) (end 162.2696 86.3601) (width 0.25) (layer F.Cu) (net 15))
 (segment (start 162.2696 86.3601) (end 161.2575 86.3601) (width 0.25) (layer F.Cu) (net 15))
 (segment (start 161.2575 86.3601) (end 160.4757 85.5783) (width 0.25) (layer F.Cu) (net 15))
 (segment (start 160.4757 85.5783) (end 160.4757 83.8083) (width 0.25) (layer F.Cu) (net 15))
 (segment (start 160.4757 83.8083) (end 161.734 82.55) (width 0.25) (layer F.Cu) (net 15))
 (segment (start 147.2634 112.5272) (end 152.4144 117.6782) (width 0.25) (layer F.Cu) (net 15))
 (segment (start 152.4144 117.6782) (end 153.9837 117.6782) (width 0.25) (layer F.Cu) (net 15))
 (segment (start 153.9837 117.6782) (end 157.7374 121.4319) (width 0.25) (layer F.Cu) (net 15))
 (segment (start 157.7374 121.4319) (end 157.7374 122.5952) (width 0.25) (layer F.Cu) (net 15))
 (segment (start 157.7374 122.5952) (end 160.2333 125.0911) (width 0.25) (layer F.Cu) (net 15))
 (segment (start 160.2333 125.0911) (end 161.5631 125.0911) (width 0.25) (layer F.Cu) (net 15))
 (segment (start 161.5631 125.0911) (end 164.0313 122.6229) (width 0.25) (layer F.Cu) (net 15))
 (segment (start 164.0313 122.6229) (end 164.0313 79.2119) (width 0.25) (layer F.Cu) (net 15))
 (segment (start 164.0313 79.2119) (end 160.5876 75.7682) (width 0.25) (layer F.Cu) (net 15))
 (segment (start 160.5876 75.7682) (end 153.226 75.7682) (width 0.25) (layer F.Cu) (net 15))
 (segment (start 161.7672 99.8982) (end 150.3744 99.8982) (width 0.25) (layer F.Cu) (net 15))
 (segment (start 150.3744 99.8982) (end 147.2634 103.0092) (width 0.25) (layer F.Cu) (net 15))
 (segment (start 147.2634 103.0092) (end 147.2634 112.5272) (width 0.25) (layer F.Cu) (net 15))
 (segment (start 147.2634 112.5272) (end 142.0813 117.7093) (width 0.25) (layer F.Cu) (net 15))
 (segment (start 142.0813 117.7093) (end 137.986 117.7093) (width 0.25) (layer F.Cu) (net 15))
 (segment (start 137.986 121.4882) (end 137.986 118.9482) (width 0.25) (layer F.Cu) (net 15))
 (segment (start 137.986 122.1076) (end 137.986 121.4882) (width 0.25) (layer F.Cu) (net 15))
 (segment (start 137.986 122.1076) (end 137.986 122.7271) (width 0.25) (layer F.Cu) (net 15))
 (segment (start 137.986 122.7271) (end 136.6801 124.033) (width 0.25) (layer F.Cu) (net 15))
 (segment (start 136.6801 124.033) (end 130.7448 124.033) (width 0.25) (layer F.Cu) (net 15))
 (segment (start 130.7448 124.033) (end 129.566 122.8542) (width 0.25) (layer F.Cu) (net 15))
 (segment (start 129.566 122.8542) (end 129.566 86.0292) (width 0.25) (layer F.Cu) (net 15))
 (segment (start 129.566 86.0292) (end 133.477 82.1182) (width 0.25) (layer F.Cu) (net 15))
 (segment (start 133.477 82.1182) (end 138.7797 82.1182) (width 0.25) (layer F.Cu) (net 15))
 (segment (start 138.7797 82.1182) (end 140.5103 80.3876) (width 0.25) (layer F.Cu) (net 15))
 (segment (start 140.5103 80.3876) (end 140.5103 80.1115) (width 0.25) (layer F.Cu) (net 15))
 (segment (start 140.5103 80.1115) (end 141.4086 79.2132) (width 0.25) (layer F.Cu) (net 15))
 (segment (start 141.4086 79.2132) (end 143.0764 79.2132) (width 0.25) (layer F.Cu) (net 15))
 (segment (start 143.0764 79.2132) (end 143.0764 73.0141) (width 0.25) (layer F.Cu) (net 15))
 (segment (start 143.0764 73.0141) (end 143.383 72.7075) (width 0.25) (layer F.Cu) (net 15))
 (segment (start 143.3713 87.63) (end 143.3713 79.5081) (width 0.25) (layer F.Cu) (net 15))
 (segment (start 143.3713 79.5081) (end 143.0764 79.2132) (width 0.25) (layer F.Cu) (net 15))
 (segment (start 160.338 109.5187) (end 161.2942 109.5187) (width 0.25) (layer F.Cu) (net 15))
 (segment (start 161.2942 109.5187) (end 161.7672 109.0457) (width 0.25) (layer F.Cu) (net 15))
 (segment (start 161.7672 109.0457) (end 161.7672 99.8982) (width 0.25) (layer F.Cu) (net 15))
 (segment (start 137.986 118.9482) (end 137.986 117.7093) (width 0.25) (layer F.Cu) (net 15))
 (segment (start 160.338 110.744) (end 160.338 109.5187) (width 0.25) (layer F.Cu) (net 15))
 (segment (start 141.796 87.63) (end 143.3713 87.63) (width 0.25) (layer F.Cu) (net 15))
 (segment (start 131.699 99.314) (end 134.9248 96.0882) (width 0.25) (layer F.Cu) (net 10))
 (segment (start 134.9248 96.0882) (end 137.986 96.0882) (width 0.25) (layer F.Cu) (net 10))
 (segment (start 137.986 101.1682) (end 137.986 102.4071) (width 0.25) (layer F.Cu) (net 12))
 (segment (start 131.826 110.808) (end 131.826 107.7923) (width 0.25) (layer F.Cu) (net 12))
 (segment (start 131.826 107.7923) (end 137.2112 102.4071) (width 0.25) (layer F.Cu) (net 12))
 (segment (start 137.2112 102.4071) (end 137.986 102.4071) (width 0.25) (layer F.Cu) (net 12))
 (segment (start 137.986 107.4871) (end 137.2112 107.4871) (width 0.25) (layer F.Cu) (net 14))
 (segment (start 137.2112 107.4871) (end 134.0239 110.6744) (width 0.25) (layer F.Cu) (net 14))
 (segment (start 134.0239 110.6744) (end 134.0239 119.7861) (width 0.25) (layer F.Cu) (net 14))
 (segment (start 134.0239 119.7861) (end 131.382 122.428) (width 0.25) (layer F.Cu) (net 14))
 (segment (start 137.986 106.2482) (end 137.986 107.4871) (width 0.25) (layer F.Cu) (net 14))
 (segment (start 137.986 98.6282) (end 137.986 99.8671) (width 0.25) (layer F.Cu) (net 11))
 (segment (start 131.826 105.156) (end 137.1149 99.8671) (width 0.25) (layer F.Cu) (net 11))
 (segment (start 137.1149 99.8671) (end 137.986 99.8671) (width 0.25) (layer F.Cu) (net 11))
 (segment (start 137.986 103.7082) (end 137.986 104.9471) (width 0.25) (layer F.Cu) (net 13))
 (segment (start 131.572 116.459) (end 133.4015 114.6295) (width 0.25) (layer F.Cu) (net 13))
 (segment (start 133.4015 114.6295) (end 133.4015 108.7568) (width 0.25) (layer F.Cu) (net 13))
 (segment (start 133.4015 108.7568) (end 137.2112 104.9471) (width 0.25) (layer F.Cu) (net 13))
 (segment (start 137.2112 104.9471) (end 137.986 104.9471) (width 0.25) (layer F.Cu) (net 13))
 (segment (start 137.986 91.0082) (end 137.986 89.7693) (width 0.25) (layer F.Cu) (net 6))
 (segment (start 137.986 89.7693) (end 138.7603 89.7693) (width 0.25) (layer F.Cu) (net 6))
 (segment (start 138.7603 89.7693) (end 140.2207 88.3089) (width 0.25) (layer F.Cu) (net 6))
 (segment (start 140.2207 88.3089) (end 140.2207 85.09) (width 0.25) (layer F.Cu) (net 6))
 (segment (start 141.796 85.09) (end 140.2207 85.09) (width 0.25) (layer F.Cu) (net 6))
 (segment (start 140.2207 85.09) (end 140.2207 82.0928) (width 0.25) (layer F.Cu) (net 6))
 (segment (start 140.2207 82.0928) (end 141.732 80.5815) (width 0.25) (layer F.Cu) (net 6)))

